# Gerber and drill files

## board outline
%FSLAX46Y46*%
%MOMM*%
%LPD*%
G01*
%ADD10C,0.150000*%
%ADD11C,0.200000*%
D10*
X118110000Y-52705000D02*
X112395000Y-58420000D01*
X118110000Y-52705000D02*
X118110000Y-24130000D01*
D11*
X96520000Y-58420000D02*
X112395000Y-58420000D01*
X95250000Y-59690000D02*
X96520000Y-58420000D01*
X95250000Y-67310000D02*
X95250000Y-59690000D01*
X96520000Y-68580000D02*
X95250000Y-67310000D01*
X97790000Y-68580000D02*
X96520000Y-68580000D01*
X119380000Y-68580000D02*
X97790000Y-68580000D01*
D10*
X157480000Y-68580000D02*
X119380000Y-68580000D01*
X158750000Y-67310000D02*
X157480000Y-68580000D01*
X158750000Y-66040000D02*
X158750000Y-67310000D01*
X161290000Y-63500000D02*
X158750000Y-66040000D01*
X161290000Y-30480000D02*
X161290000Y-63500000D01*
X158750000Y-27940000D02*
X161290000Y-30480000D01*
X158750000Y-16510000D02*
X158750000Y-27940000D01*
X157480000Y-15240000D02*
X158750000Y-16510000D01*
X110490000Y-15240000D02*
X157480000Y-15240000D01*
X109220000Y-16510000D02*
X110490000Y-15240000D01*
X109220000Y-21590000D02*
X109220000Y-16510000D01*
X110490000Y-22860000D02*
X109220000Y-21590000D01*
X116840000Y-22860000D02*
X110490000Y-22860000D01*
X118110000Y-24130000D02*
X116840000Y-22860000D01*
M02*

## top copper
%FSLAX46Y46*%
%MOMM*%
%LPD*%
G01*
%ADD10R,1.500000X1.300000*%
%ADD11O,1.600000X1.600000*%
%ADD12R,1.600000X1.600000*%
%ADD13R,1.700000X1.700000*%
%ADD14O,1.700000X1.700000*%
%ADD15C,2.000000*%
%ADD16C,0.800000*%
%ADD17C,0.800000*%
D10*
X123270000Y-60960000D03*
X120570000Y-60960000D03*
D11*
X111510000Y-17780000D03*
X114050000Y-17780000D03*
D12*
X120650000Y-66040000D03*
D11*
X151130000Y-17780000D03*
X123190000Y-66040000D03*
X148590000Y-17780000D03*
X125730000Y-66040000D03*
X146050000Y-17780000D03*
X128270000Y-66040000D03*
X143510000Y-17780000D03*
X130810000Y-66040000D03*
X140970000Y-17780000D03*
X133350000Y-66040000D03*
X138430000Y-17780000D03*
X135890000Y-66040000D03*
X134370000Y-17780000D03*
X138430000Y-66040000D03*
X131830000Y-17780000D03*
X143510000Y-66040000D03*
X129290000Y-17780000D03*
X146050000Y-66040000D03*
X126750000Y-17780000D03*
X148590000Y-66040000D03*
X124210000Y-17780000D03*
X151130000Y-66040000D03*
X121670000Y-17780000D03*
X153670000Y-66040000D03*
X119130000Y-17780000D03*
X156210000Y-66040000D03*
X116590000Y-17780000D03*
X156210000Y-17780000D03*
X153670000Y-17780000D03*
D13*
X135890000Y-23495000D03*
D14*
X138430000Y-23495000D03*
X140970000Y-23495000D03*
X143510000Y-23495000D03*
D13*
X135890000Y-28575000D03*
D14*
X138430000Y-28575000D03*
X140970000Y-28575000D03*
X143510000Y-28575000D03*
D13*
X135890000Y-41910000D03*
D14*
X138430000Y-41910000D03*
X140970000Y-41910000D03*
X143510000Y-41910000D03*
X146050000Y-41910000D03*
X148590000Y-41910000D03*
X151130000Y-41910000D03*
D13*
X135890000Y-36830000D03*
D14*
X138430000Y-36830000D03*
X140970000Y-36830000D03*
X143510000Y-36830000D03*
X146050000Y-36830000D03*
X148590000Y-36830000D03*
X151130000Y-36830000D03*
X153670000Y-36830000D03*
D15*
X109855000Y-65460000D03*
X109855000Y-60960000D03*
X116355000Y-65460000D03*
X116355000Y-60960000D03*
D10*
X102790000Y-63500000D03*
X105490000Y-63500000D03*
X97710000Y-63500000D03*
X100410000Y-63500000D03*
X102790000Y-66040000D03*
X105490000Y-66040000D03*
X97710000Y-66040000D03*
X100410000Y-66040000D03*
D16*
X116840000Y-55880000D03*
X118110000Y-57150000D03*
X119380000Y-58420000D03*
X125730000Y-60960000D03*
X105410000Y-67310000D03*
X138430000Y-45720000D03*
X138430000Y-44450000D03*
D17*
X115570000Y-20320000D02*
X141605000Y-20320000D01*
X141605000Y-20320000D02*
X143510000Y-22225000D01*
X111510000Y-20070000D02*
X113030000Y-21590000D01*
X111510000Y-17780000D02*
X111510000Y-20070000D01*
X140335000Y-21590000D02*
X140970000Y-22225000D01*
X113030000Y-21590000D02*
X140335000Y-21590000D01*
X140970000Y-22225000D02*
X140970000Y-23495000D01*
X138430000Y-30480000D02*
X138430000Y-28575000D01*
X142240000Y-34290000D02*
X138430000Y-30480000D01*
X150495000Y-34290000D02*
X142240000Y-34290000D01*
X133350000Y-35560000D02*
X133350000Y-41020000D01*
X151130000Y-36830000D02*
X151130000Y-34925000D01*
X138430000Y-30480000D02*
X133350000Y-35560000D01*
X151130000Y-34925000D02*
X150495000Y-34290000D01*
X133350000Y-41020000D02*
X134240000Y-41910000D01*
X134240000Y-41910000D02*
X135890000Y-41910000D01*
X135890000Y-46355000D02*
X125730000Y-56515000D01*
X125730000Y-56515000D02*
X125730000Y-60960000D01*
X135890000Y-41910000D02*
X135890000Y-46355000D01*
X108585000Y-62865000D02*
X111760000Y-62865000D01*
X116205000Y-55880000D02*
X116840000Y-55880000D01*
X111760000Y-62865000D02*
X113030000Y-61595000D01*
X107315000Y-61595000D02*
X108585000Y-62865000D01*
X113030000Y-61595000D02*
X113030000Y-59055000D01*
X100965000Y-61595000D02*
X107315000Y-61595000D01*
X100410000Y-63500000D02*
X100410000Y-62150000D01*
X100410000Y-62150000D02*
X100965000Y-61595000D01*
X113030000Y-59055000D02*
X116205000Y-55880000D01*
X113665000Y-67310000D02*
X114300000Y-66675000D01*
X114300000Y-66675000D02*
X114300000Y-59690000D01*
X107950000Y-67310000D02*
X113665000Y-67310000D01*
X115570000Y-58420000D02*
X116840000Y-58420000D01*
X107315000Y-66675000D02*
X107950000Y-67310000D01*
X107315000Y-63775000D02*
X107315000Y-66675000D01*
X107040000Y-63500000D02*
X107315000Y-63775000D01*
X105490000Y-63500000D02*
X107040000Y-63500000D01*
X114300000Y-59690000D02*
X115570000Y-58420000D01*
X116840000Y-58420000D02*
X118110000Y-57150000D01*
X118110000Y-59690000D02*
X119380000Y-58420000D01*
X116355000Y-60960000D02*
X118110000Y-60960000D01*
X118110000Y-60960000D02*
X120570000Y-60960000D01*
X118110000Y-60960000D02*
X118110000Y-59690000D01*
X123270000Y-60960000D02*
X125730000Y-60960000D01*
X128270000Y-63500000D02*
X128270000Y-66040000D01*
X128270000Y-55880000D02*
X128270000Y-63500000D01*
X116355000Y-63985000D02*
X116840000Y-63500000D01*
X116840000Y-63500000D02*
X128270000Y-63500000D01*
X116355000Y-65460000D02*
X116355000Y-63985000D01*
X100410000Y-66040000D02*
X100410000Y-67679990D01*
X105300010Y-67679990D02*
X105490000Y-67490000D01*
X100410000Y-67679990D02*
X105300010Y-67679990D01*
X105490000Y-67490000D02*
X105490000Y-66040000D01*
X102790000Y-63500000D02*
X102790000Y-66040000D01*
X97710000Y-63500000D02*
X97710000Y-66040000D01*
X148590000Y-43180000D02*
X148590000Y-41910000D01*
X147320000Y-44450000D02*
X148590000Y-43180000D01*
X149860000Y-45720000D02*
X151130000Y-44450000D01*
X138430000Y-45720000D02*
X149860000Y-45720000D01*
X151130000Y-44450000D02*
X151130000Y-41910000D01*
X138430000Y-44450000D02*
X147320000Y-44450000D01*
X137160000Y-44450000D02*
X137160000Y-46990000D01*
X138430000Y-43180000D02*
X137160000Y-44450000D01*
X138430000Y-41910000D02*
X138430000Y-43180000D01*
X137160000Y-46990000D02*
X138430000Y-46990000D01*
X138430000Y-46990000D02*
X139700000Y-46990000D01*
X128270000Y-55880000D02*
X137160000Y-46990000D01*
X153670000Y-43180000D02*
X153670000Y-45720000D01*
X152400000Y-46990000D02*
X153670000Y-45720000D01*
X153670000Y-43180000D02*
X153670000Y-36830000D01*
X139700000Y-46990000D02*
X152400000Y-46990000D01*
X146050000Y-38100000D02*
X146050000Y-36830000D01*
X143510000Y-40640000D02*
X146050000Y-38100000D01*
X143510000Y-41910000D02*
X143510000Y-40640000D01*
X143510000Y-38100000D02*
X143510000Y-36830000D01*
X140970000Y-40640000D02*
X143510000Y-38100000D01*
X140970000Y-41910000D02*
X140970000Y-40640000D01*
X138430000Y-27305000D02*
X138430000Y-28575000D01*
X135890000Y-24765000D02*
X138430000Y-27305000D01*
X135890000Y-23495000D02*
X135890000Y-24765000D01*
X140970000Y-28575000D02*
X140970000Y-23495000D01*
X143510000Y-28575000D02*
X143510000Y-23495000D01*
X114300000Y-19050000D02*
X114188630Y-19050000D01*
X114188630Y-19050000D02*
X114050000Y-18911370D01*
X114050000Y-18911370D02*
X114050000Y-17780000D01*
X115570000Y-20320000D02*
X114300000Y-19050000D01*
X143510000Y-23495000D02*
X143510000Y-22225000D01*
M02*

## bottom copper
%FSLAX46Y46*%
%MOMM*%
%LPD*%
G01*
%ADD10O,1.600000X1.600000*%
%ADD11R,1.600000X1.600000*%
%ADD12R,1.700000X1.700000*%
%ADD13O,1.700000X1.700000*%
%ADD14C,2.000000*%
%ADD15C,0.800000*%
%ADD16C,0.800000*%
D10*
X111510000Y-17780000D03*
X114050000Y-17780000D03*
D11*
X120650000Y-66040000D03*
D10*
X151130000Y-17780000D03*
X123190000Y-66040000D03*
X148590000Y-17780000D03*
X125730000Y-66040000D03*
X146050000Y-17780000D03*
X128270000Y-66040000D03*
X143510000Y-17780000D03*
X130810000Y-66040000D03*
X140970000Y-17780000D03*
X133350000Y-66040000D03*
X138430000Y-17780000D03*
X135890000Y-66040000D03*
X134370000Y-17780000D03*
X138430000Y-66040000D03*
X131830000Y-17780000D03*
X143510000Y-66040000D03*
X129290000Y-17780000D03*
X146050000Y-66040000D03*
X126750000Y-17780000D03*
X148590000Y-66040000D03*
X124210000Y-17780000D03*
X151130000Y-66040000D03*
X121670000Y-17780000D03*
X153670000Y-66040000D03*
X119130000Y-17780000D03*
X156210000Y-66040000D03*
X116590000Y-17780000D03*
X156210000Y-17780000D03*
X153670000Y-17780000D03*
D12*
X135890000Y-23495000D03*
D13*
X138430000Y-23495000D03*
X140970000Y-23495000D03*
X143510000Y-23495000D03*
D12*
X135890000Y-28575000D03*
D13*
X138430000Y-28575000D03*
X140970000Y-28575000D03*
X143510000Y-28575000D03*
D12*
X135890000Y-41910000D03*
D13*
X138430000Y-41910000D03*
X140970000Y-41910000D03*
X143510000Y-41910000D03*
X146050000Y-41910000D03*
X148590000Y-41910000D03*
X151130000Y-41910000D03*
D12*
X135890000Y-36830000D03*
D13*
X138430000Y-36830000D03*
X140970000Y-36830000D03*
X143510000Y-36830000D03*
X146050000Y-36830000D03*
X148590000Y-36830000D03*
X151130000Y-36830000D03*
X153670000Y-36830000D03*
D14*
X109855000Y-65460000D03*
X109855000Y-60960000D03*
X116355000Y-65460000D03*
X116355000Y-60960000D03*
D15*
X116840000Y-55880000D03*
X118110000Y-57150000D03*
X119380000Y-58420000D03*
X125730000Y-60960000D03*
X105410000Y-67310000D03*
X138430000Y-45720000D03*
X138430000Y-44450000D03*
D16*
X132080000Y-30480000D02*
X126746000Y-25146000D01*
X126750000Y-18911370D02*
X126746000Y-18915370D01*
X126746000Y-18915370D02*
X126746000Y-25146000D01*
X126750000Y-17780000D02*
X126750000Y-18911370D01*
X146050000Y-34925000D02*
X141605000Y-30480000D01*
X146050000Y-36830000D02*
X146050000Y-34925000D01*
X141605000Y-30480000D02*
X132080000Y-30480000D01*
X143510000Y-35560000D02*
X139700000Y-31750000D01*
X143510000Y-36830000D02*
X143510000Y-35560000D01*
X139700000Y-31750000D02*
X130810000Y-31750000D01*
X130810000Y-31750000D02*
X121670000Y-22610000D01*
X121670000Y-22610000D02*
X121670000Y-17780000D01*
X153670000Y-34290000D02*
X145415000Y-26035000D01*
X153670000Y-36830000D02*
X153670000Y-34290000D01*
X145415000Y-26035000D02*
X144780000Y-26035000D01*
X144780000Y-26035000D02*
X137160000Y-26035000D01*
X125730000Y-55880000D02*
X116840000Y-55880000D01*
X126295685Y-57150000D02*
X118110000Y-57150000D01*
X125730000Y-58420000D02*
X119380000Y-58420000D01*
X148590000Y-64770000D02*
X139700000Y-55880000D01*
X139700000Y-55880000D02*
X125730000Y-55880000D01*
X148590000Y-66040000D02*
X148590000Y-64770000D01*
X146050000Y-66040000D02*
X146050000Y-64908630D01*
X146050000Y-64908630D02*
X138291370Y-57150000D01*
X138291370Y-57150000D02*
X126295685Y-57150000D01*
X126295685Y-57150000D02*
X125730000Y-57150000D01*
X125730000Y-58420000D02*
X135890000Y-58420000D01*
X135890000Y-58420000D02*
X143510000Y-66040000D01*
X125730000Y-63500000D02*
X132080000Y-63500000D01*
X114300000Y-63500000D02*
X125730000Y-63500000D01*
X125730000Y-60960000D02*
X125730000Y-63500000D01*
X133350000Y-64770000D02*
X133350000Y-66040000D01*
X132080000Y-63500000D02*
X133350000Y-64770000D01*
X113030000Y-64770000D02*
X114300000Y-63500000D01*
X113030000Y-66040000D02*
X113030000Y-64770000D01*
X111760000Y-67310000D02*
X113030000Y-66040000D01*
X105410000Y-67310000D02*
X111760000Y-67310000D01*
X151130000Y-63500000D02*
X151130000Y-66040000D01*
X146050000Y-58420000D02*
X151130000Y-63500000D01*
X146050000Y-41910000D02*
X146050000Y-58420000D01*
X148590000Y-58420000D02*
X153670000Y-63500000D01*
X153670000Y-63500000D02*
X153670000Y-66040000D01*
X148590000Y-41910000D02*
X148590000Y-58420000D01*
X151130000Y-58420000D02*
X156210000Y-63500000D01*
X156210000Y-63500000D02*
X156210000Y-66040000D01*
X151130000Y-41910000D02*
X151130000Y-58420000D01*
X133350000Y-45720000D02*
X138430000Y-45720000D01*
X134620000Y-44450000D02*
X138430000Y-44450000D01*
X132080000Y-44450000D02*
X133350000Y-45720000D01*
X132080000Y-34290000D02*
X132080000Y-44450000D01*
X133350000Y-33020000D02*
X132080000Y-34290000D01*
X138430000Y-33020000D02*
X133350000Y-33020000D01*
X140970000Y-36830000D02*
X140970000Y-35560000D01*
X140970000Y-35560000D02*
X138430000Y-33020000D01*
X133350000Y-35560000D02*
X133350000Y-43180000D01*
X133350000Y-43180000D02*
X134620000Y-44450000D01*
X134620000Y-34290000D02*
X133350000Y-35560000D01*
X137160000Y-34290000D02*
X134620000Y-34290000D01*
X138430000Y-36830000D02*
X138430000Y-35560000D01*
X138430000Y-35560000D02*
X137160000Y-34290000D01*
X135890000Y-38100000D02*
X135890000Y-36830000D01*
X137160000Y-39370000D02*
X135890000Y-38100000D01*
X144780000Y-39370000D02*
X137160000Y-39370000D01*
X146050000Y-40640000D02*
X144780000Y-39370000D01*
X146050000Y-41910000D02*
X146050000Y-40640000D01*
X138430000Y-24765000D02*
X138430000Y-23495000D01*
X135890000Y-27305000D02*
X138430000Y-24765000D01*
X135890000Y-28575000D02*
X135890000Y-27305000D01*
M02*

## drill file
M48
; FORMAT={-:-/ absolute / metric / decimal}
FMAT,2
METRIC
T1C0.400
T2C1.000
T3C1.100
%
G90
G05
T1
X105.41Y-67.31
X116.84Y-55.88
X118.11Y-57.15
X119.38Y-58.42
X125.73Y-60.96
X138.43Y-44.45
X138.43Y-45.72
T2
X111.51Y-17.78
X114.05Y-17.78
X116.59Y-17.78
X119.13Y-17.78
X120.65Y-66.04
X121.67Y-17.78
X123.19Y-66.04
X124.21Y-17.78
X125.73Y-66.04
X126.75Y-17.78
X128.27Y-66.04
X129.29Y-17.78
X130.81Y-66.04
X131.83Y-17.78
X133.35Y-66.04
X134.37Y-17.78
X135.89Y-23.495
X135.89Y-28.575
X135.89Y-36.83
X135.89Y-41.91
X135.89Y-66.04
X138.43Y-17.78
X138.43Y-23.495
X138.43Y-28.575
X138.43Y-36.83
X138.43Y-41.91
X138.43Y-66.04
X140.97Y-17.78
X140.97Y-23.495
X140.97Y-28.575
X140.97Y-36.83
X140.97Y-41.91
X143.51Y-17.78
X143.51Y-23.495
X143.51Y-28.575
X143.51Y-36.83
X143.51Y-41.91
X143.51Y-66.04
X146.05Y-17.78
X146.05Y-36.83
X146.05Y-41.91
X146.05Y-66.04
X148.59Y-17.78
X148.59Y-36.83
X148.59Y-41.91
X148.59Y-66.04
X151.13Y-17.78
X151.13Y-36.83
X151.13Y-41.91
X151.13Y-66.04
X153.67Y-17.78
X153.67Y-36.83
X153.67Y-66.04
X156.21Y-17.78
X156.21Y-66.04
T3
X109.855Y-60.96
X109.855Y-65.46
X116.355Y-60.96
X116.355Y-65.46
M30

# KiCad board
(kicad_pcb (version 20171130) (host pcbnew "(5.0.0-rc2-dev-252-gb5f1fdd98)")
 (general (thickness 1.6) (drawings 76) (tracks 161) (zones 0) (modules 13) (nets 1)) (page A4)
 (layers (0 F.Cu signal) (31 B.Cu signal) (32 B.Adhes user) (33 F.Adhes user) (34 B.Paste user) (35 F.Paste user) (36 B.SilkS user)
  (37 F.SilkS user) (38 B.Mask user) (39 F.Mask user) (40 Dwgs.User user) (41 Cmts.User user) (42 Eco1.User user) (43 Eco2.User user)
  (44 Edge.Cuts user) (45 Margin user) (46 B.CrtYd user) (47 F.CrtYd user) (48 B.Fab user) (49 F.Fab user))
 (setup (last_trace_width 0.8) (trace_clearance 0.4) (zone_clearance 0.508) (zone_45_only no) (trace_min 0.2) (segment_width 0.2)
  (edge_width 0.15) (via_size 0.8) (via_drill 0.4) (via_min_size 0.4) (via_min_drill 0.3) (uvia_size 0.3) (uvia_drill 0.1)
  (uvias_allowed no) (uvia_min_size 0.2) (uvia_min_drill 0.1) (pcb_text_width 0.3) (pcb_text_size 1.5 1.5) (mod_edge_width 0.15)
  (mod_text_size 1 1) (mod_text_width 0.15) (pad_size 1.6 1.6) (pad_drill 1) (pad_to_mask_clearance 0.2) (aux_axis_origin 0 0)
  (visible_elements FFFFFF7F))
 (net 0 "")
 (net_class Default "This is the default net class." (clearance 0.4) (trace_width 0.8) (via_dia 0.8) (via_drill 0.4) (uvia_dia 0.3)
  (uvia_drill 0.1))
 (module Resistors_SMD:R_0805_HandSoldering (layer F.Cu) (at 121.92 60.96)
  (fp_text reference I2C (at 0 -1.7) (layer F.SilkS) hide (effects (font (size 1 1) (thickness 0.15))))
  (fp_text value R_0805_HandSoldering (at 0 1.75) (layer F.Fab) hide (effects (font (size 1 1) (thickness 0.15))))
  (pad 2 smd rect (at 1.35 0) (size 1.5 1.3) (layers F.Cu F.Paste F.Mask))
  (pad 1 smd rect (at -1.35 0) (size 1.5 1.3) (layers F.Cu F.Paste F.Mask)))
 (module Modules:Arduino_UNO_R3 (layer B.Cu) (at 120.65 66.04)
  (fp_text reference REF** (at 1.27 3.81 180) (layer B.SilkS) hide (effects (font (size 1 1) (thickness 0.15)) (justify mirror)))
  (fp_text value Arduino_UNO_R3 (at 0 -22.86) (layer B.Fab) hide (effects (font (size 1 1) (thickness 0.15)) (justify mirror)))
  (pad 32 thru_hole oval (at -9.14 -48.26 270) (size 1.6 1.6) (drill 1) (layers *.Cu *.Mask))
  (pad 31 thru_hole oval (at -6.6 -48.26 270) (size 1.6 1.6) (drill 1) (layers *.Cu *.Mask))
  (pad 1 thru_hole rect (at 0 0 270) (size 1.6 1.6) (drill 1) (layers *.Cu *.Mask))
  (pad 17 thru_hole oval (at 30.48 -48.26 270) (size 1.6 1.6) (drill 1) (layers *.Cu *.Mask))
  (pad 2 thru_hole oval (at 2.54 0 270) (size 1.6 1.6) (drill 1) (layers *.Cu *.Mask))
  (pad 18 thru_hole oval (at 27.94 -48.26 270) (size 1.6 1.6) (drill 1) (layers *.Cu *.Mask))
  (pad 3 thru_hole oval (at 5.08 0 270) (size 1.6 1.6) (drill 1) (layers *.Cu *.Mask))
  (pad 19 thru_hole oval (at 25.4 -48.26 270) (size 1.6 1.6) (drill 1) (layers *.Cu *.Mask))
  (pad 4 thru_hole oval (at 7.62 0 270) (size 1.6 1.6) (drill 1) (layers *.Cu *.Mask))
  (pad 20 thru_hole oval (at 22.86 -48.26 270) (size 1.6 1.6) (drill 1) (layers *.Cu *.Mask))
  (pad 5 thru_hole oval (at 10.16 0 270) (size 1.6 1.6) (drill 1) (layers *.Cu *.Mask))
  (pad 21 thru_hole oval (at 20.32 -48.26 270) (size 1.6 1.6) (drill 1) (layers *.Cu *.Mask))
  (pad 6 thru_hole oval (at 12.7 0 270) (size 1.6 1.6) (drill 1) (layers *.Cu *.Mask))
  (pad 22 thru_hole oval (at 17.78 -48.26 270) (size 1.6 1.6) (drill 1) (layers *.Cu *.Mask))
  (pad 7 thru_hole oval (at 15.24 0 270) (size 1.6 1.6) (drill 1) (layers *.Cu *.Mask))
  (pad 23 thru_hole oval (at 13.72 -48.26 270) (size 1.6 1.6) (drill 1) (layers *.Cu *.Mask))
  (pad 8 thru_hole oval (at 17.78 0 270) (size 1.6 1.6) (drill 1) (layers *.Cu *.Mask))
  (pad 24 thru_hole oval (at 11.18 -48.26 270) (size 1.6 1.6) (drill 1) (layers *.Cu *.Mask))
  (pad 9 thru_hole oval (at 22.86 0 270) (size 1.6 1.6) (drill 1) (layers *.Cu *.Mask))
  (pad 25 thru_hole oval (at 8.64 -48.26 270) (size 1.6 1.6) (drill 1) (layers *.Cu *.Mask))
  (pad 10 thru_hole oval (at 25.4 0 270) (size 1.6 1.6) (drill 1) (layers *.Cu *.Mask))
  (pad 26 thru_hole oval (at 6.1 -48.26 270) (size 1.6 1.6) (drill 1) (layers *.Cu *.Mask))
  (pad 11 thru_hole oval (at 27.94 0 270) (size 1.6 1.6) (drill 1) (layers *.Cu *.Mask))
  (pad 27 thru_hole oval (at 3.56 -48.26 270) (size 1.6 1.6) (drill 1) (layers *.Cu *.Mask))
  (pad 12 thru_hole oval (at 30.48 0 270) (size 1.6 1.6) (drill 1) (layers *.Cu *.Mask))
  (pad 28 thru_hole oval (at 1.02 -48.26 270) (size 1.6 1.6) (drill 1) (layers *.Cu *.Mask))
  (pad 13 thru_hole oval (at 33.02 0 270) (size 1.6 1.6) (drill 1) (layers *.Cu *.Mask))
  (pad 29 thru_hole oval (at -1.52 -48.26 270) (size 1.6 1.6) (drill 1) (layers *.Cu *.Mask))
  (pad 14 thru_hole oval (at 35.56 0 270) (size 1.6 1.6) (drill 1) (layers *.Cu *.Mask))
  (pad 30 thru_hole oval (at -4.06 -48.26 270) (size 1.6 1.6) (drill 1) (layers *.Cu *.Mask))
  (pad 15 thru_hole oval (at 35.56 -48.26 270) (size 1.6 1.6) (drill 1) (layers *.Cu *.Mask))
  (pad 16 thru_hole oval (at 33.02 -48.26 270) (size 1.6 1.6) (drill 1) (layers *.Cu *.Mask)))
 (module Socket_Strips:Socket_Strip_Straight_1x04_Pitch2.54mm (layer F.Cu) (at 135.89 23.495 90)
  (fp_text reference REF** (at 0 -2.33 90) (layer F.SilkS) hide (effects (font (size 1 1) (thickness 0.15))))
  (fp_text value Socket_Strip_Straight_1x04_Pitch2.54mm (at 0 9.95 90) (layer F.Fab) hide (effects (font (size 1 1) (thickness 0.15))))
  (pad 1 thru_hole rect (at 0 0 90) (size 1.7 1.7) (drill 1) (layers *.Cu *.Mask))
  (pad 2 thru_hole oval (at 0 2.54 90) (size 1.7 1.7) (drill 1) (layers *.Cu *.Mask))
  (pad 3 thru_hole oval (at 0 5.08 90) (size 1.7 1.7) (drill 1) (layers *.Cu *.Mask))
  (pad 4 thru_hole oval (at 0 7.62 90) (size 1.7 1.7) (drill 1) (layers *.Cu *.Mask)))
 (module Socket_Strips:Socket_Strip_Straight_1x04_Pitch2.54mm (layer F.Cu) (at 135.89 28.575 90)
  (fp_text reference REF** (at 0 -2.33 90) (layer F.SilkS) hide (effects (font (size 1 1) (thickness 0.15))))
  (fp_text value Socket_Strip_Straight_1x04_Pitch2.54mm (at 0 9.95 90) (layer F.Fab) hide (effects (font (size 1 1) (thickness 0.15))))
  (pad 1 thru_hole rect (at 0 0 90) (size 1.7 1.7) (drill 1) (layers *.Cu *.Mask))
  (pad 2 thru_hole oval (at 0 2.54 90) (size 1.7 1.7) (drill 1) (layers *.Cu *.Mask))
  (pad 3 thru_hole oval (at 0 5.08 90) (size 1.7 1.7) (drill 1) (layers *.Cu *.Mask))
  (pad 4 thru_hole oval (at 0 7.62 90) (size 1.7 1.7) (drill 1) (layers *.Cu *.Mask)))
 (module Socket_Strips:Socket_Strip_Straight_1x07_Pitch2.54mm (layer F.Cu) (at 135.89 41.91 90)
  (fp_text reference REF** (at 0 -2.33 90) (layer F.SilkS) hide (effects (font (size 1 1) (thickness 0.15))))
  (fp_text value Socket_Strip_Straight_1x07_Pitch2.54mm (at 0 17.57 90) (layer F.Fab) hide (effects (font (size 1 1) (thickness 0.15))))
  (pad 1 thru_hole rect (at 0 0 90) (size 1.7 1.7) (drill 1) (layers *.Cu *.Mask))
  (pad 2 thru_hole oval (at 0 2.54 90) (size 1.7 1.7) (drill 1) (layers *.Cu *.Mask))
  (pad 3 thru_hole oval (at 0 5.08 90) (size 1.7 1.7) (drill 1) (layers *.Cu *.Mask))
  (pad 4 thru_hole oval (at 0 7.62 90) (size 1.7 1.7) (drill 1) (layers *.Cu *.Mask))
  (pad 5 thru_hole oval (at 0 10.16 90) (size 1.7 1.7) (drill 1) (layers *.Cu *.Mask))
  (pad 6 thru_hole oval (at 0 12.7 90) (size 1.7 1.7) (drill 1) (layers *.Cu *.Mask))
  (pad 7 thru_hole oval (at 0 15.24 90) (size 1.7 1.7) (drill 1) (layers *.Cu *.Mask)))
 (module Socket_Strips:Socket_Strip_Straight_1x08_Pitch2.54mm (layer F.Cu) (at 135.89 36.83 90)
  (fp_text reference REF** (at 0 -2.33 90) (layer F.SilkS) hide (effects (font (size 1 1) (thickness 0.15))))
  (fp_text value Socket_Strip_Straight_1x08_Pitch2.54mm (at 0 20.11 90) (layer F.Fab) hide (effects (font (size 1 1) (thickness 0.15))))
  (pad 1 thru_hole rect (at 0 0 90) (size 1.7 1.7) (drill 1) (layers *.Cu *.Mask))
  (pad 2 thru_hole oval (at 0 2.54 90) (size 1.7 1.7) (drill 1) (layers *.Cu *.Mask))
  (pad 3 thru_hole oval (at 0 5.08 90) (size 1.7 1.7) (drill 1) (layers *.Cu *.Mask))
  (pad 4 thru_hole oval (at 0 7.62 90) (size 1.7 1.7) (drill 1) (layers *.Cu *.Mask))
  (pad 5 thru_hole oval (at 0 10.16 90) (size 1.7 1.7) (drill 1) (layers *.Cu *.Mask))
  (pad 6 thru_hole oval (at 0 12.7 90) (size 1.7 1.7) (drill 1) (layers *.Cu *.Mask))
  (pad 7 thru_hole oval (at 0 15.24 90) (size 1.7 1.7) (drill 1) (layers *.Cu *.Mask))
  (pad 8 thru_hole oval (at 0 17.78 90) (size 1.7 1.7) (drill 1) (layers *.Cu *.Mask)))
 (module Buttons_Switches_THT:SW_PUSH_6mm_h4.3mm (layer F.Cu) (at 109.855 60.96)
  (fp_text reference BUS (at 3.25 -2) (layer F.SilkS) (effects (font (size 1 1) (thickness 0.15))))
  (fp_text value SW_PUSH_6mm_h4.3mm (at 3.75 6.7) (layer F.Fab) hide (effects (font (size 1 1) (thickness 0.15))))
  (pad 2 thru_hole circle (at 0 4.5 90) (size 2 2) (drill 1.1) (layers *.Cu *.Mask))
  (pad 1 thru_hole circle (at 0 0 90) (size 2 2) (drill 1.1) (layers *.Cu *.Mask))
  (pad 2 thru_hole circle (at 6.5 4.5 90) (size 2 2) (drill 1.1) (layers *.Cu *.Mask))
  (pad 1 thru_hole circle (at 6.5 0 90) (size 2 2) (drill 1.1) (layers *.Cu *.Mask)))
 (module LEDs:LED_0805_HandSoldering (layer F.Cu) (at 104.14 63.5)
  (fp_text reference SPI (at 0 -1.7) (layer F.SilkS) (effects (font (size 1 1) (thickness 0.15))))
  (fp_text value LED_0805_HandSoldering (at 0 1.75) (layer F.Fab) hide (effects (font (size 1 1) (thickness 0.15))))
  (pad 1 smd rect (at -1.35 0) (size 1.5 1.3) (layers F.Cu F.Paste F.Mask))
  (pad 2 smd rect (at 1.35 0) (size 1.5 1.3) (layers F.Cu F.Paste F.Mask)))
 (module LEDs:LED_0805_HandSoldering (layer F.Cu) (at 99.06 63.5)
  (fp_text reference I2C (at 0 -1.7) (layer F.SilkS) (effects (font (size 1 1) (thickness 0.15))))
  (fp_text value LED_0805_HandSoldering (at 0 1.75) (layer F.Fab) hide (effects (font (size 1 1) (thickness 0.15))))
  (pad 1 smd rect (at -1.35 0) (size 1.5 1.3) (layers F.Cu F.Paste F.Mask))
  (pad 2 smd rect (at 1.35 0) (size 1.5 1.3) (layers F.Cu F.Paste F.Mask)))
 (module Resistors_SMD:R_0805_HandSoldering (layer F.Cu) (at 104.14 66.04)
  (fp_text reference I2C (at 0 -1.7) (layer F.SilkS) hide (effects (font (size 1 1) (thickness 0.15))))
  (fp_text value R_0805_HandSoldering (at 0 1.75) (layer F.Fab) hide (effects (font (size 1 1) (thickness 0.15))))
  (pad 1 smd rect (at -1.35 0) (size 1.5 1.3) (layers F.Cu F.Paste F.Mask))
  (pad 2 smd rect (at 1.35 0) (size 1.5 1.3) (layers F.Cu F.Paste F.Mask)))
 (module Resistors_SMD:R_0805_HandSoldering (layer F.Cu) (at 99.06 66.04)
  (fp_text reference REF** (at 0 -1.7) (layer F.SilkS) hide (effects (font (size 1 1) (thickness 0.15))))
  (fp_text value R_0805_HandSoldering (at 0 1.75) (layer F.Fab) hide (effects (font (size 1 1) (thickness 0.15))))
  (pad 1 smd rect (at -1.35 0) (size 1.5 1.3) (layers F.Cu F.Paste F.Mask))
  (pad 2 smd rect (at 1.35 0) (size 1.5 1.3) (layers F.Cu F.Paste F.Mask)))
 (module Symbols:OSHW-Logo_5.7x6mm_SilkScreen (layer F.Cu) (at 121.285 29.21 90)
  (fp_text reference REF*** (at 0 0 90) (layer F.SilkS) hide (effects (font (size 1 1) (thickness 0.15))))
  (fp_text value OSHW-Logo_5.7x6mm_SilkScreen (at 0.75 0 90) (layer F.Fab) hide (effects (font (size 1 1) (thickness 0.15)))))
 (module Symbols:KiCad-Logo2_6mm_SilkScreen (layer F.Cu) (at 121.285 42.545 90)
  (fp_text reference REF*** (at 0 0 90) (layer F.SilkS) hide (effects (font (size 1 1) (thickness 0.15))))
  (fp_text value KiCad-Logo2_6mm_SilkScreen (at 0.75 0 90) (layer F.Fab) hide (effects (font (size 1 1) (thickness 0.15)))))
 (gr_line (start 118.11 52.705) (end 112.395 58.42) (layer Edge.Cuts) (width 0.15))
 (gr_line (start 118.11 52.705) (end 118.11 24.13) (layer Edge.Cuts) (width 0.15))
 (gr_line (start 96.52 58.42) (end 112.395 58.42) (layer Edge.Cuts) (width 0.2))
 (gr_line (start 95.25 59.69) (end 96.52 58.42) (layer Edge.Cuts) (width 0.2))
 (gr_line (start 95.25 67.31) (end 95.25 59.69) (layer Edge.Cuts) (width 0.2))
 (gr_line (start 96.52 68.58) (end 95.25 67.31) (layer Edge.Cuts) (width 0.2))
 (gr_line (start 97.79 68.58) (end 96.52 68.58) (layer Edge.Cuts) (width 0.2))
 (gr_line (start 119.38 68.58) (end 97.79 68.58) (layer Edge.Cuts) (width 0.2))
 (gr_line (start 157.48 68.58) (end 119.38 68.58) (layer Edge.Cuts) (width 0.15))
 (gr_line (start 158.75 67.31) (end 157.48 68.58) (layer Edge.Cuts) (width 0.15))
 (gr_line (start 158.75 66.04) (end 158.75 67.31) (layer Edge.Cuts) (width 0.15))
 (gr_line (start 161.29 63.5) (end 158.75 66.04) (layer Edge.Cuts) (width 0.15))
 (gr_line (start 161.29 30.48) (end 161.29 63.5) (layer Edge.Cuts) (width 0.15))
 (gr_line (start 158.75 27.94) (end 161.29 30.48) (layer Edge.Cuts) (width 0.15))
 (gr_line (start 158.75 16.51) (end 158.75 27.94) (layer Edge.Cuts) (width 0.15))
 (gr_line (start 157.48 15.24) (end 158.75 16.51) (layer Edge.Cuts) (width 0.15))
 (gr_line (start 110.49 15.24) (end 157.48 15.24) (layer Edge.Cuts) (width 0.15))
 (gr_line (start 109.22 16.51) (end 110.49 15.24) (layer Edge.Cuts) (width 0.15))
 (gr_line (start 109.22 21.59) (end 109.22 16.51) (layer Edge.Cuts) (width 0.15))
 (gr_line (start 110.49 22.86) (end 109.22 21.59) (layer Edge.Cuts) (width 0.15))
 (gr_line (start 116.84 22.86) (end 110.49 22.86) (layer Edge.Cuts) (width 0.15))
 (gr_line (start 118.11 24.13) (end 116.84 22.86) (layer Edge.Cuts) (width 0.15))
 (segment (start 132.08 30.48) (end 126.746 25.146) (width 0.8) (layer B.Cu) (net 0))
 (segment (start 126.75 18.91137) (end 126.746 18.91537) (width 0.8) (layer B.Cu) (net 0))
 (segment (start 126.746 18.91537) (end 126.746 25.146) (width 0.8) (layer B.Cu) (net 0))
 (segment (start 126.75 17.78) (end 126.75 18.91137) (width 0.8) (layer B.Cu) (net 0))
 (segment (start 146.05 34.925) (end 141.605 30.48) (width 0.8) (layer B.Cu) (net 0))
 (segment (start 146.05 36.83) (end 146.05 34.925) (width 0.8) (layer B.Cu) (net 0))
 (segment (start 141.605 30.48) (end 132.08 30.48) (width 0.8) (layer B.Cu) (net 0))
 (segment (start 143.51 35.56) (end 139.7 31.75) (width 0.8) (layer B.Cu) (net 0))
 (segment (start 143.51 36.83) (end 143.51 35.56) (width 0.8) (layer B.Cu) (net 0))
 (segment (start 139.7 31.75) (end 130.81 31.75) (width 0.8) (layer B.Cu) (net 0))
 (segment (start 130.81 31.75) (end 121.67 22.61) (width 0.8) (layer B.Cu) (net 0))
 (segment (start 121.67 22.61) (end 121.67 17.78) (width 0.8) (layer B.Cu) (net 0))
 (segment (start 153.67 34.29) (end 145.415 26.035) (width 0.8) (layer B.Cu) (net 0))
 (segment (start 153.67 36.83) (end 153.67 34.29) (width 0.8) (layer B.Cu) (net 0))
 (segment (start 145.415 26.035) (end 144.78 26.035) (width 0.8) (layer B.Cu) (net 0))
 (segment (start 144.78 26.035) (end 137.16 26.035) (width 0.8) (layer B.Cu) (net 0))
 (segment (start 115.57 20.32) (end 141.605 20.32) (width 0.8) (layer F.Cu) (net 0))
 (segment (start 141.605 20.32) (end 143.51 22.225) (width 0.8) (layer F.Cu) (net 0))
 (segment (start 111.51 20.07) (end 113.03 21.59) (width 0.8) (layer F.Cu) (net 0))
 (segment (start 111.51 17.78) (end 111.51 20.07) (width 0.8) (layer F.Cu) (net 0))
 (segment (start 140.335 21.59) (end 140.97 22.225) (width 0.8) (layer F.Cu) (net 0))
 (segment (start 113.03 21.59) (end 140.335 21.59) (width 0.8) (layer F.Cu) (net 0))
 (segment (start 140.97 22.225) (end 140.97 23.495) (width 0.8) (layer F.Cu) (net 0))
 (segment (start 138.43 30.48) (end 138.43 28.575) (width 0.8) (layer F.Cu) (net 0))
 (segment (start 142.24 34.29) (end 138.43 30.48) (width 0.8) (layer F.Cu) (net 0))
 (segment (start 150.495 34.29) (end 142.24 34.29) (width 0.8) (layer F.Cu) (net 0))
 (segment (start 133.35 35.56) (end 133.35 41.02) (width 0.8) (layer F.Cu) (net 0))
 (segment (start 151.13 36.83) (end 151.13 34.925) (width 0.8) (layer F.Cu) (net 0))
 (segment (start 138.43 30.48) (end 133.35 35.56) (width 0.8) (layer F.Cu) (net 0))
 (segment (start 151.13 34.925) (end 150.495 34.29) (width 0.8) (layer F.Cu) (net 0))
 (segment (start 133.35 41.02) (end 134.24 41.91) (width 0.8) (layer F.Cu) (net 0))
 (segment (start 134.24 41.91) (end 135.89 41.91) (width 0.8) (layer F.Cu) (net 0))
 (segment (start 135.89 46.355) (end 125.73 56.515) (width 0.8) (layer F.Cu) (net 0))
 (segment (start 125.73 56.515) (end 125.73 60.96) (width 0.8) (layer F.Cu) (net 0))
 (segment (start 135.89 41.91) (end 135.89 46.355) (width 0.8) (layer F.Cu) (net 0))
 (segment (start 125.73 55.88) (end 116.84 55.88) (width 0.8) (layer B.Cu) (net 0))
 (segment (start 126.295685 57.15) (end 118.11 57.15) (width 0.8) (layer B.Cu) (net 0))
 (segment (start 125.73 58.42) (end 119.38 58.42) (width 0.8) (layer B.Cu) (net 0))
 (segment (start 148.59 64.77) (end 139.7 55.88) (width 0.8) (layer B.Cu) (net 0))
 (segment (start 139.7 55.88) (end 125.73 55.88) (width 0.8) (layer B.Cu) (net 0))
 (segment (start 148.59 66.04) (end 148.59 64.77) (width 0.8) (layer B.Cu) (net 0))
 (segment (start 146.05 66.04) (end 146.05 64.90863) (width 0.8) (layer B.Cu) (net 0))
 (segment (start 146.05 64.90863) (end 138.29137 57.15) (width 0.8) (layer B.Cu) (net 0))
 (segment (start 138.29137 57.15) (end 126.295685 57.15) (width 0.8) (layer B.Cu) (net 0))
 (segment (start 126.295685 57.15) (end 125.73 57.15) (width 0.8) (layer B.Cu) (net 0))
 (via (at 116.84 55.88) (size 0.8) (drill 0.4) (layers F.Cu B.Cu) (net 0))
 (via (at 118.11 57.15) (size 0.8) (drill 0.4) (layers F.Cu B.Cu) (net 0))
 (segment (start 108.585 62.865) (end 111.76 62.865) (width 0.8) (layer F.Cu) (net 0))
 (segment (start 116.205 55.88) (end 116.84 55.88) (width 0.8) (layer F.Cu) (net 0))
 (segment (start 111.76 62.865) (end 113.03 61.595) (width 0.8) (layer F.Cu) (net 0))
 (segment (start 107.315 61.595) (end 108.585 62.865) (width 0.8) (layer F.Cu) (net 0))
 (segment (start 113.03 61.595) (end 113.03 59.055) (width 0.8) (layer F.Cu) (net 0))
 (segment (start 100.965 61.595) (end 107.315 61.595) (width 0.8) (layer F.Cu) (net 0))
 (segment (start 100.41 63.5) (end 100.41 62.15) (width 0.8) (layer F.Cu) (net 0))
 (segment (start 100.41 62.15) (end 100.965 61.595) (width 0.8) (layer F.Cu) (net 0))
 (segment (start 113.03 59.055) (end 116.205 55.88) (width 0.8) (layer F.Cu) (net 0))
 (segment (start 113.665 67.31) (end 114.3 66.675) (width 0.8) (layer F.Cu) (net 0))
 (segment (start 114.3 66.675) (end 114.3 59.69) (width 0.8) (layer F.Cu) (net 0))
 (segment (start 107.95 67.31) (end 113.665 67.31) (width 0.8) (layer F.Cu) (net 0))
 (segment (start 115.57 58.42) (end 116.84 58.42) (width 0.8) (layer F.Cu) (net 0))
 (segment (start 107.315 66.675) (end 107.95 67.31) (width 0.8) (layer F.Cu) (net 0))
 (segment (start 107.315 63.775) (end 107.315 66.675) (width 0.8) (layer F.Cu) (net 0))
 (segment (start 107.04 63.5) (end 107.315 63.775) (width 0.8) (layer F.Cu) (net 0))
 (segment (start 105.49 63.5) (end 107.04 63.5) (width 0.8) (layer F.Cu) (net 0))
 (segment (start 114.3 59.69) (end 115.57 58.42) (width 0.8) (layer F.Cu) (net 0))
 (segment (start 116.84 58.42) (end 118.11 57.15) (width 0.8) (layer F.Cu) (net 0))
 (segment (start 125.73 58.42) (end 135.89 58.42) (width 0.8) (layer B.Cu) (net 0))
 (segment (start 135.89 58.42) (end 143.51 66.04) (width 0.8) (layer B.Cu) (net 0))
 (segment (start 118.11 59.69) (end 119.38 58.42) (width 0.8) (layer F.Cu) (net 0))
 (segment (start 116.355 60.96) (end 118.11 60.96) (width 0.8) (layer F.Cu) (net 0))
 (segment (start 118.11 60.96) (end 120.57 60.96) (width 0.8) (layer F.Cu) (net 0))
 (segment (start 118.11 60.96) (end 118.11 59.69) (width 0.8) (layer F.Cu) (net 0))
 (via (at 119.38 58.42) (size 0.8) (drill 0.4) (layers F.Cu B.Cu) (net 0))
 (segment (start 125.73 63.5) (end 132.08 63.5) (width 0.8) (layer B.Cu) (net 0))
 (segment (start 114.3 63.5) (end 125.73 63.5) (width 0.8) (layer B.Cu) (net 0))
 (segment (start 125.73 60.96) (end 125.73 63.5) (width 0.8) (layer B.Cu) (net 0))
 (via (at 125.73 60.96) (size 0.8) (drill 0.4) (layers F.Cu B.Cu) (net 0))
 (segment (start 123.27 60.96) (end 125.73 60.96) (width 0.8) (layer F.Cu) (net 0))
 (segment (start 128.27 63.5) (end 128.27 66.04) (width 0.8) (layer F.Cu) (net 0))
 (segment (start 128.27 55.88) (end 128.27 63.5) (width 0.8) (layer F.Cu) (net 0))
 (segment (start 116.355 63.985) (end 116.84 63.5) (width 0.8) (layer F.Cu) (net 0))
 (segment (start 116.84 63.5) (end 128.27 63.5) (width 0.8) (layer F.Cu) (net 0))
 (segment (start 116.355 65.46) (end 116.355 63.985) (width 0.8) (layer F.Cu) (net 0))
 (segment (start 133.35 64.77) (end 133.35 66.04) (width 0.8) (layer B.Cu) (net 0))
 (segment (start 132.08 63.5) (end 133.35 64.77) (width 0.8) (layer B.Cu) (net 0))
 (segment (start 113.03 64.77) (end 114.3 63.5) (width 0.8) (layer B.Cu) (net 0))
 (segment (start 113.03 66.04) (end 113.03 64.77) (width 0.8) (layer B.Cu) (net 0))
 (segment (start 111.76 67.31) (end 113.03 66.04) (width 0.8) (layer B.Cu) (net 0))
 (segment (start 105.41 67.31) (end 111.76 67.31) (width 0.8) (layer B.Cu) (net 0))
 (via (at 105.41 67.31) (size 0.8) (drill 0.4) (layers F.Cu B.Cu) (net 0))
 (segment (start 100.41 66.04) (end 100.41 67.67999) (width 0.8) (layer F.Cu) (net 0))
 (segment (start 105.30001 67.67999) (end 105.49 67.49) (width 0.8) (layer F.Cu) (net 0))
 (segment (start 100.41 67.67999) (end 105.30001 67.67999) (width 0.8) (layer F.Cu) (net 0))
 (segment (start 105.49 67.49) (end 105.49 66.04) (width 0.8) (layer F.Cu) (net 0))
 (segment (start 102.79 63.5) (end 102.79 66.04) (width 0.8) (layer F.Cu) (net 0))
 (segment (start 97.71 63.5) (end 97.71 66.04) (width 0.8) (layer F.Cu) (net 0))
 (segment (start 151.13 63.5) (end 151.13 66.04) (width 0.8) (layer B.Cu) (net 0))
 (segment (start 146.05 58.42) (end 151.13 63.5) (width 0.8) (layer B.Cu) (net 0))
 (segment (start 146.05 41.91) (end 146.05 58.42) (width 0.8) (layer B.Cu) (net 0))
 (segment (start 148.59 58.42) (end 153.67 63.5) (width 0.8) (layer B.Cu) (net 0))
 (segment (start 153.67 63.5) (end 153.67 66.04) (width 0.8) (layer B.Cu) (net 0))
 (segment (start 148.59 41.91) (end 148.59 58.42) (width 0.8) (layer B.Cu) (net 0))
 (segment (start 151.13 58.42) (end 156.21 63.5) (width 0.8) (layer B.Cu) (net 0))
 (segment (start 156.21 63.5) (end 156.21 66.04) (width 0.8) (layer B.Cu) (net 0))
 (segment (start 151.13 41.91) (end 151.13 58.42) (width 0.8) (layer B.Cu) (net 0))
 (segment (start 148.59 43.18) (end 148.59 41.91) (width 0.8) (layer F.Cu) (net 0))
 (segment (start 147.32 44.45) (end 148.59 43.18) (width 0.8) (layer F.Cu) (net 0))
 (segment (start 149.86 45.72) (end 151.13 44.45) (width 0.8) (layer F.Cu) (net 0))
 (segment (start 138.43 45.72) (end 149.86 45.72) (width 0.8) (layer F.Cu) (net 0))
 (segment (start 151.13 44.45) (end 151.13 41.91) (width 0.8) (layer F.Cu) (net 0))
 (segment (start 138.43 44.45) (end 147.32 44.45) (width 0.8) (layer F.Cu) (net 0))
 (segment (start 133.35 45.72) (end 138.43 45.72) (width 0.8) (layer B.Cu) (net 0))
 (segment (start 134.62 44.45) (end 138.43 44.45) (width 0.8) (layer B.Cu) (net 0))
 (via (at 138.43 45.72) (size 0.8) (drill 0.4) (layers F.Cu B.Cu) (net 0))
 (via (at 138.43 44.45) (size 0.8) (drill 0.4) (layers F.Cu B.Cu) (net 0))
 (segment (start 137.16 44.45) (end 137.16 46.99) (width 0.8) (layer F.Cu) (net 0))
 (segment (start 138.43 43.18) (end 137.16 44.45) (width 0.8) (layer F.Cu) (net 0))
 (segment (start 138.43 41.91) (end 138.43 43.18) (width 0.8) (layer F.Cu) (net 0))
 (segment (start 137.16 46.99) (end 138.43 46.99) (width 0.8) (layer F.Cu) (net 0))
 (segment (start 138.43 46.99) (end 139.7 46.99) (width 0.8) (layer F.Cu) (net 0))
 (segment (start 128.27 55.88) (end 137.16 46.99) (width 0.8) (layer F.Cu) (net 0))
 (segment (start 153.67 43.18) (end 153.67 45.72) (width 0.8) (layer F.Cu) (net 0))
 (segment (start 152.4 46.99) (end 153.67 45.72) (width 0.8) (layer F.Cu) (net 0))
 (segment (start 153.67 43.18) (end 153.67 36.83) (width 0.8) (layer F.Cu) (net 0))
 (segment (start 139.7 46.99) (end 152.4 46.99) (width 0.8) (layer F.Cu) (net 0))
 (segment (start 132.08 44.45) (end 133.35 45.72) (width 0.8) (layer B.Cu) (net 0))
 (segment (start 132.08 34.29) (end 132.08 44.45) (width 0.8) (layer B.Cu) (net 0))
 (segment (start 133.35 33.02) (end 132.08 34.29) (width 0.8) (layer B.Cu) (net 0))
 (segment (start 138.43 33.02) (end 133.35 33.02) (width 0.8) (layer B.Cu) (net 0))
 (segment (start 140.97 36.83) (end 140.97 35.56) (width 0.8) (layer B.Cu) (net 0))
 (segment (start 140.97 35.56) (end 138.43 33.02) (width 0.8) (layer B.Cu) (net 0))
 (segment (start 133.35 35.56) (end 133.35 43.18) (width 0.8) (layer B.Cu) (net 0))
 (segment (start 133.35 43.18) (end 134.62 44.45) (width 0.8) (layer B.Cu) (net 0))
 (segment (start 134.62 34.29) (end 133.35 35.56) (width 0.8) (layer B.Cu) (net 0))
 (segment (start 137.16 34.29) (end 134.62 34.29) (width 0.8) (layer B.Cu) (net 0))
 (segment (start 138.43 36.83) (end 138.43 35.56) (width 0.8) (layer B.Cu) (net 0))
 (segment (start 138.43 35.56) (end 137.16 34.29) (width 0.8) (layer B.Cu) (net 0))
 (segment (start 135.89 38.1) (end 135.89 36.83) (width 0.8) (layer B.Cu) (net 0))
 (segment (start 137.16 39.37) (end 135.89 38.1) (width 0.8) (layer B.Cu) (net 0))
 (segment (start 144.78 39.37) (end 137.16 39.37) (width 0.8) (layer B.Cu) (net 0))
 (segment (start 146.05 40.64) (end 144.78 39.37) (width 0.8) (layer B.Cu) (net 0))
 (segment (start 146.05 41.91) (end 146.05 40.64) (width 0.8) (layer B.Cu) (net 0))
 (segment (start 146.05 38.1) (end 146.05 36.83) (width 0.8) (layer F.Cu) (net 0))
 (segment (start 143.51 40.64) (end 146.05 38.1) (width 0.8) (layer F.Cu) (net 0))
 (segment (start 143.51 41.91) (end 143.51 40.64) (width 0.8) (layer F.Cu) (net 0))
 (segment (start 143.51 38.1) (end 143.51 36.83) (width 0.8) (layer F.Cu) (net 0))
 (segment (start 140.97 40.64) (end 143.51 38.1) (width 0.8) (layer F.Cu) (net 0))
 (segment (start 140.97 41.91) (end 140.97 40.64) (width 0.8) (layer F.Cu) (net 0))
 (segment (start 138.43 27.305) (end 138.43 28.575) (width 0.8) (layer F.Cu) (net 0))
 (segment (start 135.89 24.765) (end 138.43 27.305) (width 0.8) (layer F.Cu) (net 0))
 (segment (start 135.89 23.495) (end 135.89 24.765) (width 0.8) (layer F.Cu) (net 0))
 (segment (start 138.43 24.765) (end 138.43 23.495) (width 0.8) (layer B.Cu) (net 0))
 (segment (start 135.89 27.305) (end 138.43 24.765) (width 0.8) (layer B.Cu) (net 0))
 (segment (start 135.89 28.575) (end 135.89 27.305) (width 0.8) (layer B.Cu) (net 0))
 (segment (start 140.97 28.575) (end 140.97 23.495) (width 0.8) (layer F.Cu) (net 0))
 (segment (start 143.51 28.575) (end 143.51 23.495) (width 0.8) (layer F.Cu) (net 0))
 (segment (start 114.3 19.05) (end 114.18863 19.05) (width 0.8) (layer F.Cu) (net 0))
 (segment (start 114.18863 19.05) (end 114.05 18.91137) (width 0.8) (layer F.Cu) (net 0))
 (segment (start 114.05 18.91137) (end 114.05 17.78) (width 0.8) (layer F.Cu) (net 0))
 (segment (start 115.57 20.32) (end 114.3 19.05) (width 0.8) (layer F.Cu) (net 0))
 (segment (start 143.51 23.495) (end 143.51 22.225) (width 0.8) (layer F.Cu) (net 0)))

